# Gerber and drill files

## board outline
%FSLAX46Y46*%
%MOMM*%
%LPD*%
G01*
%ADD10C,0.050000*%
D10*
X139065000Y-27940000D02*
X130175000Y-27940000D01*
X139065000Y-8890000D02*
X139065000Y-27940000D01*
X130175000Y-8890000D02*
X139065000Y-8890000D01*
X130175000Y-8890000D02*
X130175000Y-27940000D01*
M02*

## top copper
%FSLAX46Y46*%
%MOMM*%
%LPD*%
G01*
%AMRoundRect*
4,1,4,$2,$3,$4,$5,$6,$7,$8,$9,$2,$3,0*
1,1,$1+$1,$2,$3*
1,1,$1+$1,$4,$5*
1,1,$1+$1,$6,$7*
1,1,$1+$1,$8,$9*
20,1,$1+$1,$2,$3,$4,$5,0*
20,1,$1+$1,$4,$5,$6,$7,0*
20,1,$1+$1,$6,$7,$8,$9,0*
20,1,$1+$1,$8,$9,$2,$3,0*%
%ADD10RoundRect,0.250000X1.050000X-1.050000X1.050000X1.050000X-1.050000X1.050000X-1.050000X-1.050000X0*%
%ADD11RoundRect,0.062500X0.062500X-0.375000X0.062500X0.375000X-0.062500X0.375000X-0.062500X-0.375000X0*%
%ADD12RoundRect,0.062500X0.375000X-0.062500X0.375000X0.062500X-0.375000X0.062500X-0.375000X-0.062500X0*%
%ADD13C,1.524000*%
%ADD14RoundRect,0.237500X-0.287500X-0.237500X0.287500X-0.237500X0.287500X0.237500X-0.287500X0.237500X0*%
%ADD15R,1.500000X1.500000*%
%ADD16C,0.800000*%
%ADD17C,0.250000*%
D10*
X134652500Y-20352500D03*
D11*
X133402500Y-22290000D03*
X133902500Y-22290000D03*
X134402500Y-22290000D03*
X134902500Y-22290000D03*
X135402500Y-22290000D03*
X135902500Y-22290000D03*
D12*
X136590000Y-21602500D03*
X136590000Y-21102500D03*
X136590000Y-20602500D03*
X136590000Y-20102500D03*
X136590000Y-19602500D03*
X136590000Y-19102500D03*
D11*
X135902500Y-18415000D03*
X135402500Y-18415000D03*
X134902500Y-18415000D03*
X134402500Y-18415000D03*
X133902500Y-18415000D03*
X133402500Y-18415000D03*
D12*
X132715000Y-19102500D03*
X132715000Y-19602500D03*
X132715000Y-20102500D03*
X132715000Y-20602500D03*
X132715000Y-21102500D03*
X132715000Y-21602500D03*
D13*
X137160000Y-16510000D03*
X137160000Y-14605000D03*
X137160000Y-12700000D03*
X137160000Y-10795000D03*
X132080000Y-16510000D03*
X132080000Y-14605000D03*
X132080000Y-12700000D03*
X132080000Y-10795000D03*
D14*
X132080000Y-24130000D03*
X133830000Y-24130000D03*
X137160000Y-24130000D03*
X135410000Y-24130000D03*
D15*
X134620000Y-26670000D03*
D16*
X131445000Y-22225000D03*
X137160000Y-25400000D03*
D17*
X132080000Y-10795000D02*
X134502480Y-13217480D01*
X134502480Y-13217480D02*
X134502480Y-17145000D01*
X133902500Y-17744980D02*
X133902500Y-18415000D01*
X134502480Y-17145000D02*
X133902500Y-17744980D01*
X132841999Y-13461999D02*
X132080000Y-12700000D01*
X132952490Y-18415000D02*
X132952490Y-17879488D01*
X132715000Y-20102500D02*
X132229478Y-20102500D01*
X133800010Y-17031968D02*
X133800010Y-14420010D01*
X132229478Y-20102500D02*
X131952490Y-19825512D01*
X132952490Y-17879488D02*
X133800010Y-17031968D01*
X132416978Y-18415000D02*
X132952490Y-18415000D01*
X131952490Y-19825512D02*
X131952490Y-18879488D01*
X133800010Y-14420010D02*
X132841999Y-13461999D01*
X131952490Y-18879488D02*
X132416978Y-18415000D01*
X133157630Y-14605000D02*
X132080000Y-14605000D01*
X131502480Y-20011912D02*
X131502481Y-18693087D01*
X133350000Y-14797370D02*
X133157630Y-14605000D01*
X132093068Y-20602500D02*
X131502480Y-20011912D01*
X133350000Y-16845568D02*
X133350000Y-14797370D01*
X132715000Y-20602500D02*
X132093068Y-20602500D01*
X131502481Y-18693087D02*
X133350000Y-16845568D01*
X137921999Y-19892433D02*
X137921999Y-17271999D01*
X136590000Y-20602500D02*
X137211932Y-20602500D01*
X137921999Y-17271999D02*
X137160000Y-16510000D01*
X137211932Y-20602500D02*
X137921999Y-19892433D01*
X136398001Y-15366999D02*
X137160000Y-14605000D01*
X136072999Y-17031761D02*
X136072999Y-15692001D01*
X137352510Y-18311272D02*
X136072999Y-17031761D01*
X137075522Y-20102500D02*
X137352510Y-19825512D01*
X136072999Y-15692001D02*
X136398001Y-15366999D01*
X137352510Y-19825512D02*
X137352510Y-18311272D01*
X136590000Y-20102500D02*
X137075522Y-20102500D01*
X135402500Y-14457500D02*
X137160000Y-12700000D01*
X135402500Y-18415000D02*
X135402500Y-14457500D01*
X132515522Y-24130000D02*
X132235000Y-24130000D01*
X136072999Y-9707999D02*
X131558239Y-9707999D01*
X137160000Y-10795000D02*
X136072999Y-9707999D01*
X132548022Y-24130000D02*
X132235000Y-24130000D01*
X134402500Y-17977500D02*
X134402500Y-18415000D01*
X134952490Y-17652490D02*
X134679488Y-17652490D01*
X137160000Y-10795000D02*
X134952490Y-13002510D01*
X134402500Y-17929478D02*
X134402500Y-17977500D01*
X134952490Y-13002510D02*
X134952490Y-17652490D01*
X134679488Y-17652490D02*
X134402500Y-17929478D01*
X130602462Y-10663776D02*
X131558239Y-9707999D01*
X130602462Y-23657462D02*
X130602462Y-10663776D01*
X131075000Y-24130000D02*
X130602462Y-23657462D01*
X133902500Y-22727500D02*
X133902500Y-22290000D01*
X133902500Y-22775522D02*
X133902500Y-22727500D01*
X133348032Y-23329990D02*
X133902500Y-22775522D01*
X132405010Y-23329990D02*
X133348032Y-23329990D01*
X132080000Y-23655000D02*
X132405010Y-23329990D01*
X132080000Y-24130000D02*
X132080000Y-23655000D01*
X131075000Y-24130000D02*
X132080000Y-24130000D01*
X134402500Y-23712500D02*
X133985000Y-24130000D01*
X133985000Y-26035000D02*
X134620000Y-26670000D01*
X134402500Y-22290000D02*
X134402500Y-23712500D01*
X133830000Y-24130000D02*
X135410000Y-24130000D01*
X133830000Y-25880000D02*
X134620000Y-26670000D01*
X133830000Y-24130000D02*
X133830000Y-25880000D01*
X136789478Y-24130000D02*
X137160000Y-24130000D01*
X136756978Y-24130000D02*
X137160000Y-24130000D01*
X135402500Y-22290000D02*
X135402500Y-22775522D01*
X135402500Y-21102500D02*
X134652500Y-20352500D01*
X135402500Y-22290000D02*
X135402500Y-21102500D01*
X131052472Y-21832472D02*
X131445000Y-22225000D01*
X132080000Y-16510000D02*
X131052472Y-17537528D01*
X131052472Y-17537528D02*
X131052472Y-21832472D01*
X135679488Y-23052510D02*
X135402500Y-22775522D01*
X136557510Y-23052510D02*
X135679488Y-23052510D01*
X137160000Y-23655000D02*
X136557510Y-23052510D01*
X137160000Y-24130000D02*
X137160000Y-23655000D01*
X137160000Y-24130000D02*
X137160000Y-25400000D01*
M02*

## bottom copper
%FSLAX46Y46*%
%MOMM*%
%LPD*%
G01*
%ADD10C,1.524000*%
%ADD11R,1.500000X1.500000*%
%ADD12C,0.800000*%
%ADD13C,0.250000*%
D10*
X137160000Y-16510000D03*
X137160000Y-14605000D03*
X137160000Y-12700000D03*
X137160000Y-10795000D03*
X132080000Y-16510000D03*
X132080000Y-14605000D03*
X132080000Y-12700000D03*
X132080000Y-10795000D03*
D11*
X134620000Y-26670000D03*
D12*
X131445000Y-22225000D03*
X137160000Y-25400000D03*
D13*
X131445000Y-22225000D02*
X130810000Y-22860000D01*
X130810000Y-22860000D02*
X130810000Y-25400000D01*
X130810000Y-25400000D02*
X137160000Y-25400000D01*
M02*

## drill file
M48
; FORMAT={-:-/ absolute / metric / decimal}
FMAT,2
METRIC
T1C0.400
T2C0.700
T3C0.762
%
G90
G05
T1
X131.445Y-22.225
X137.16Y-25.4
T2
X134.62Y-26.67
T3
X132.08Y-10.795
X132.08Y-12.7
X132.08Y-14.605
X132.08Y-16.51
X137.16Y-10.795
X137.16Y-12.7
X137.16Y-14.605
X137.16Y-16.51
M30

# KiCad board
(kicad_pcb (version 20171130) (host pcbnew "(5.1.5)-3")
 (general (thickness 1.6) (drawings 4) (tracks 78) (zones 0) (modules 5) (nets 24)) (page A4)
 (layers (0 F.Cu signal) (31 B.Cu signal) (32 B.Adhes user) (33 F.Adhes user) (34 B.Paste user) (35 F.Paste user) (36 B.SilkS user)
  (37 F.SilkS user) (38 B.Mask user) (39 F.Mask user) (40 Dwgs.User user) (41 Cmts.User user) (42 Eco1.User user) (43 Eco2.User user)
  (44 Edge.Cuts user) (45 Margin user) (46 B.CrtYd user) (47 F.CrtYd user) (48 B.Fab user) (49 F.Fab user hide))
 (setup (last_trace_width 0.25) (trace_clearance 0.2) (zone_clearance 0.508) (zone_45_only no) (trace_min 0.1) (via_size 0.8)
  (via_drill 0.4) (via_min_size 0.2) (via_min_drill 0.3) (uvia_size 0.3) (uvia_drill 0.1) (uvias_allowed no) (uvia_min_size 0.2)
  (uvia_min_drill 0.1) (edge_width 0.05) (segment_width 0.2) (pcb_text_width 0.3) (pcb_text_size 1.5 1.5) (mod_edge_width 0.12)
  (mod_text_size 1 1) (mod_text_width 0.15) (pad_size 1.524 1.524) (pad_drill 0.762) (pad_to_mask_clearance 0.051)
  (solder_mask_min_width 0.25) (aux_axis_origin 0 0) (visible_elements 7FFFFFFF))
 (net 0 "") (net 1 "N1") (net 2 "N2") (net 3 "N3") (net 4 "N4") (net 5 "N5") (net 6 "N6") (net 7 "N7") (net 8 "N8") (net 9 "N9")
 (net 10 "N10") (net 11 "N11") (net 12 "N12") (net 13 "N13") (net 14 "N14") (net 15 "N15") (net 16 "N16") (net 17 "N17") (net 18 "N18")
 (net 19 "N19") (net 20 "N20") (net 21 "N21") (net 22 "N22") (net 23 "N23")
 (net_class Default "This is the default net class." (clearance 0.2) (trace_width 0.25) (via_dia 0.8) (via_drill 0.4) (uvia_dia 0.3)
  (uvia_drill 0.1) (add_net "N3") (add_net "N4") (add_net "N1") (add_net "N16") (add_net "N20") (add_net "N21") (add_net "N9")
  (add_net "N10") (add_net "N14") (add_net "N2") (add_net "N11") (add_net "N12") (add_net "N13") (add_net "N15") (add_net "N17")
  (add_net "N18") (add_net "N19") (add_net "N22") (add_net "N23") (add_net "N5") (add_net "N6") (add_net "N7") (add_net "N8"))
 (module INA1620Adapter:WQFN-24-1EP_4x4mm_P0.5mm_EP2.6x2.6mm (layer F.Cu) (at 134.6525 20.3525 90)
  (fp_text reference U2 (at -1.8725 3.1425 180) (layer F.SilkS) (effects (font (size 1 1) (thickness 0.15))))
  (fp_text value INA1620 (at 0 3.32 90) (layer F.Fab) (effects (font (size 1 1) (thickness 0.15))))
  (pad 25 smd roundrect (at 0 0 90) (size 2.6 2.6) (layers F.Cu F.Mask) (roundrect_rratio 0.096154) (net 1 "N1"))
  (pad "" smd roundrect (at -0.65 -0.65 90) (size 1.05 1.05) (layers F.Paste) (roundrect_rratio 0.238095))
  (pad "" smd roundrect (at -0.65 0.65 90) (size 1.05 1.05) (layers F.Paste) (roundrect_rratio 0.238095))
  (pad "" smd roundrect (at 0.65 -0.65 90) (size 1.05 1.05) (layers F.Paste) (roundrect_rratio 0.238095))
  (pad "" smd roundrect (at 0.65 0.65 90) (size 1.05 1.05) (layers F.Paste) (roundrect_rratio 0.238095))
  (pad 1 smd roundrect (at -1.9375 -1.25 90) (size 0.875 0.25) (layers F.Cu F.Paste F.Mask) (roundrect_rratio 0.25) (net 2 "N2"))
  (pad 2 smd roundrect (at -1.9375 -0.75 90) (size 0.875 0.25) (layers F.Cu F.Paste F.Mask) (roundrect_rratio 0.25) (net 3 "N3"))
  (pad 3 smd roundrect (at -1.9375 -0.25 90) (size 0.875 0.25) (layers F.Cu F.Paste F.Mask) (roundrect_rratio 0.25) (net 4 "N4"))
  (pad 4 smd roundrect (at -1.9375 0.25 90) (size 0.875 0.25) (layers F.Cu F.Paste F.Mask) (roundrect_rratio 0.25) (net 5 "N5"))
  (pad 5 smd roundrect (at -1.9375 0.75 90) (size 0.875 0.25) (layers F.Cu F.Paste F.Mask) (roundrect_rratio 0.25) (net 1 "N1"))
  (pad 6 smd roundrect (at -1.9375 1.25 90) (size 0.875 0.25) (layers F.Cu F.Paste F.Mask) (roundrect_rratio 0.25) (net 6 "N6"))
  (pad 7 smd roundrect (at -1.25 1.9375 90) (size 0.25 0.875) (layers F.Cu F.Paste F.Mask) (roundrect_rratio 0.25) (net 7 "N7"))
  (pad 8 smd roundrect (at -0.75 1.9375 90) (size 0.25 0.875) (layers F.Cu F.Paste F.Mask) (roundrect_rratio 0.25) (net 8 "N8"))
  (pad 9 smd roundrect (at -0.25 1.9375 90) (size 0.25 0.875) (layers F.Cu F.Paste F.Mask) (roundrect_rratio 0.25) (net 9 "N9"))
  (pad 10 smd roundrect (at 0.25 1.9375 90) (size 0.25 0.875) (layers F.Cu F.Paste F.Mask) (roundrect_rratio 0.25) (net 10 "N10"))
  (pad 11 smd roundrect (at 0.75 1.9375 90) (size 0.25 0.875) (layers F.Cu F.Paste F.Mask) (roundrect_rratio 0.25) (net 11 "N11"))
  (pad 12 smd roundrect (at 1.25 1.9375 90) (size 0.25 0.875) (layers F.Cu F.Paste F.Mask) (roundrect_rratio 0.25) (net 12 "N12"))
  (pad 13 smd roundrect (at 1.9375 1.25 90) (size 0.875 0.25) (layers F.Cu F.Paste F.Mask) (roundrect_rratio 0.25) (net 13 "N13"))
  (pad 14 smd roundrect (at 1.9375 0.75 90) (size 0.875 0.25) (layers F.Cu F.Paste F.Mask) (roundrect_rratio 0.25) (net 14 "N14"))
  (pad 15 smd roundrect (at 1.9375 0.25 90) (size 0.875 0.25) (layers F.Cu F.Paste F.Mask) (roundrect_rratio 0.25) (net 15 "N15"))
  (pad 16 smd roundrect (at 1.9375 -0.25 90) (size 0.875 0.25) (layers F.Cu F.Paste F.Mask) (roundrect_rratio 0.25) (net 3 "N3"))
  (pad 17 smd roundrect (at 1.9375 -0.75 90) (size 0.875 0.25) (layers F.Cu F.Paste F.Mask) (roundrect_rratio 0.25) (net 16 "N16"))
  (pad 18 smd roundrect (at 1.9375 -1.25 90) (size 0.875 0.25) (layers F.Cu F.Paste F.Mask) (roundrect_rratio 0.25) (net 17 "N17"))
  (pad 19 smd roundrect (at 1.25 -1.9375 90) (size 0.25 0.875) (layers F.Cu F.Paste F.Mask) (roundrect_rratio 0.25) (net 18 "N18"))
  (pad 20 smd roundrect (at 0.75 -1.9375 90) (size 0.25 0.875) (layers F.Cu F.Paste F.Mask) (roundrect_rratio 0.25) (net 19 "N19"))
  (pad 21 smd roundrect (at 0.25 -1.9375 90) (size 0.25 0.875) (layers F.Cu F.Paste F.Mask) (roundrect_rratio 0.25) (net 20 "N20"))
  (pad 22 smd roundrect (at -0.25 -1.9375 90) (size 0.25 0.875) (layers F.Cu F.Paste F.Mask) (roundrect_rratio 0.25) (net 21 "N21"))
  (pad 23 smd roundrect (at -0.75 -1.9375 90) (size 0.25 0.875) (layers F.Cu F.Paste F.Mask) (roundrect_rratio 0.25) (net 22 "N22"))
  (pad 24 smd roundrect (at -1.25 -1.9375 90) (size 0.25 0.875) (layers F.Cu F.Paste F.Mask) (roundrect_rratio 0.25) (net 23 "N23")))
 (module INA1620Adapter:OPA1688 (layer F.Cu) (at 134.62 13.97)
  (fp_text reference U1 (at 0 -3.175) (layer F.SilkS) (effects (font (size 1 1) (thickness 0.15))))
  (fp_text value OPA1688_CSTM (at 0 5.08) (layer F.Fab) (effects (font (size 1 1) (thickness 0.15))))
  (pad 5 thru_hole circle (at 2.54 2.54) (size 1.524 1.524) (drill 0.762) (layers *.Cu *.Mask) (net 9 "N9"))
  (pad 6 thru_hole circle (at 2.54 0.635) (size 1.524 1.524) (drill 0.762) (layers *.Cu *.Mask) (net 10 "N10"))
  (pad 7 thru_hole circle (at 2.54 -1.27) (size 1.524 1.524) (drill 0.762) (layers *.Cu *.Mask) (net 14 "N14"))
  (pad 8 thru_hole circle (at 2.54 -3.175) (size 1.524 1.524) (drill 0.762) (layers *.Cu *.Mask) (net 3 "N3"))
  (pad 4 thru_hole circle (at -2.54 2.54) (size 1.524 1.524) (drill 0.762) (layers *.Cu *.Mask) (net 1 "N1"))
  (pad 3 thru_hole circle (at -2.54 0.635) (size 1.524 1.524) (drill 0.762) (layers *.Cu *.Mask) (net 21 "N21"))
  (pad 2 thru_hole circle (at -2.54 -1.27) (size 1.524 1.524) (drill 0.762) (layers *.Cu *.Mask) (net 20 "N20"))
  (pad 1 thru_hole circle (at -2.54 -3.175) (size 1.524 1.524) (drill 0.762) (layers *.Cu *.Mask) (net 16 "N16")))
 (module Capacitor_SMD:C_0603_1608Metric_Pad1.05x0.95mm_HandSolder (layer F.Cu) (at 132.955 24.13)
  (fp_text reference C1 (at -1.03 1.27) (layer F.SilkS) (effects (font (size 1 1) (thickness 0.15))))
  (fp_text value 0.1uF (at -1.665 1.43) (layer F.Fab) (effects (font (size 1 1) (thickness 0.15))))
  (pad 1 smd roundrect (at -0.875 0) (size 1.05 0.95) (layers F.Cu F.Paste F.Mask) (roundrect_rratio 0.25) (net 3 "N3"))
  (pad 2 smd roundrect (at 0.875 0) (size 1.05 0.95) (layers F.Cu F.Paste F.Mask) (roundrect_rratio 0.25) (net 4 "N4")))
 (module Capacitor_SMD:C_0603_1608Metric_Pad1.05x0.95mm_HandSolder (layer F.Cu) (at 136.285 24.13)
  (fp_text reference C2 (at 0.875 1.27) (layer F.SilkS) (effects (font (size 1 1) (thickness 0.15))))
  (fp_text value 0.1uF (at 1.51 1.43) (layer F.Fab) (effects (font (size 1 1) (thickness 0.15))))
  (pad 2 smd roundrect (at 0.875 0) (size 1.05 0.95) (layers F.Cu F.Paste F.Mask) (roundrect_rratio 0.25) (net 1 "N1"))
  (pad 1 smd roundrect (at -0.875 0) (size 1.05 0.95) (layers F.Cu F.Paste F.Mask) (roundrect_rratio 0.25) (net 4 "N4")))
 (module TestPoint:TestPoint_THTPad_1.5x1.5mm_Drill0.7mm (layer F.Cu) (at 134.62 26.67)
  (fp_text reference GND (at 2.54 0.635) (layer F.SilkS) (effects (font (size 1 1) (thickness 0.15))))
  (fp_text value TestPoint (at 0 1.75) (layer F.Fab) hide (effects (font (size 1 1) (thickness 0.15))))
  (pad 1 thru_hole rect (at 0 0) (size 1.5 1.5) (drill 0.7) (layers *.Cu *.Mask) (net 4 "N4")))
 (gr_line (start 139.065 27.94) (end 130.175 27.94) (layer Edge.Cuts) (width 0.05))
 (gr_line (start 139.065 8.89) (end 139.065 27.94) (layer Edge.Cuts) (width 0.05))
 (gr_line (start 130.175 8.89) (end 139.065 8.89) (layer Edge.Cuts) (width 0.05))
 (gr_line (start 130.175 8.89) (end 130.175 27.94) (layer Edge.Cuts) (width 0.05))
 (segment (start 132.08 10.795) (end 134.50248 13.21748) (width 0.25) (layer F.Cu) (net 16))
 (segment (start 134.50248 13.21748) (end 134.50248 17.145) (width 0.25) (layer F.Cu) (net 16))
 (segment (start 133.9025 17.74498) (end 133.9025 18.415) (width 0.25) (layer F.Cu) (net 16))
 (segment (start 134.50248 17.145) (end 133.9025 17.74498) (width 0.25) (layer F.Cu) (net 16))
 (segment (start 132.841999 13.461999) (end 132.08 12.7) (width 0.25) (layer F.Cu) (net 20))
 (segment (start 132.95249 18.415) (end 132.95249 17.879488) (width 0.25) (layer F.Cu) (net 20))
 (segment (start 132.715 20.1025) (end 132.229478 20.1025) (width 0.25) (layer F.Cu) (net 20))
 (segment (start 133.80001 17.031968) (end 133.80001 14.42001) (width 0.25) (layer F.Cu) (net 20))
 (segment (start 132.229478 20.1025) (end 131.95249 19.825512) (width 0.25) (layer F.Cu) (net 20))
 (segment (start 132.95249 17.879488) (end 133.80001 17.031968) (width 0.25) (layer F.Cu) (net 20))
 (segment (start 132.416978 18.415) (end 132.95249 18.415) (width 0.25) (layer F.Cu) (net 20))
 (segment (start 131.95249 19.825512) (end 131.95249 18.879488) (width 0.25) (layer F.Cu) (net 20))
 (segment (start 133.80001 14.42001) (end 132.841999 13.461999) (width 0.25) (layer F.Cu) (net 20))
 (segment (start 131.95249 18.879488) (end 132.416978 18.415) (width 0.25) (layer F.Cu) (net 20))
 (segment (start 133.15763 14.605) (end 132.08 14.605) (width 0.25) (layer F.Cu) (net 21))
 (segment (start 131.50248 20.011912) (end 131.502481 18.693087) (width 0.25) (layer F.Cu) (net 21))
 (segment (start 133.35 14.79737) (end 133.15763 14.605) (width 0.25) (layer F.Cu) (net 21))
 (segment (start 132.093068 20.6025) (end 131.50248 20.011912) (width 0.25) (layer F.Cu) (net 21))
 (segment (start 133.35 16.845568) (end 133.35 14.79737) (width 0.25) (layer F.Cu) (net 21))
 (segment (start 132.715 20.6025) (end 132.093068 20.6025) (width 0.25) (layer F.Cu) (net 21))
 (segment (start 131.502481 18.693087) (end 133.35 16.845568) (width 0.25) (layer F.Cu) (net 21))
 (segment (start 137.921999 19.892433) (end 137.921999 17.271999) (width 0.25) (layer F.Cu) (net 9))
 (segment (start 136.59 20.6025) (end 137.211932 20.6025) (width 0.25) (layer F.Cu) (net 9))
 (segment (start 137.921999 17.271999) (end 137.16 16.51) (width 0.25) (layer F.Cu) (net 9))
 (segment (start 137.211932 20.6025) (end 137.921999 19.892433) (width 0.25) (layer F.Cu) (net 9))
 (segment (start 136.398001 15.366999) (end 137.16 14.605) (width 0.25) (layer F.Cu) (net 10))
 (segment (start 136.072999 17.031761) (end 136.072999 15.692001) (width 0.25) (layer F.Cu) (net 10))
 (segment (start 137.35251 18.311272) (end 136.072999 17.031761) (width 0.25) (layer F.Cu) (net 10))
 (segment (start 137.075522 20.1025) (end 137.35251 19.825512) (width 0.25) (layer F.Cu) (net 10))
 (segment (start 136.072999 15.692001) (end 136.398001 15.366999) (width 0.25) (layer F.Cu) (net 10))
 (segment (start 137.35251 19.825512) (end 137.35251 18.311272) (width 0.25) (layer F.Cu) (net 10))
 (segment (start 136.59 20.1025) (end 137.075522 20.1025) (width 0.25) (layer F.Cu) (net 10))
 (segment (start 135.4025 14.4575) (end 137.16 12.7) (width 0.25) (layer F.Cu) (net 14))
 (segment (start 135.4025 18.415) (end 135.4025 14.4575) (width 0.25) (layer F.Cu) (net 14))
 (segment (start 132.515522 24.13) (end 132.235 24.13) (width 0.25) (layer F.Cu) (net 3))
 (segment (start 136.072999 9.707999) (end 131.558239 9.707999) (width 0.25) (layer F.Cu) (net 3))
 (segment (start 137.16 10.795) (end 136.072999 9.707999) (width 0.25) (layer F.Cu) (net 3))
 (segment (start 132.548022 24.13) (end 132.235 24.13) (width 0.25) (layer F.Cu) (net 3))
 (segment (start 134.4025 17.9775) (end 134.4025 18.415) (width 0.25) (layer F.Cu) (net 3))
 (segment (start 134.95249 17.65249) (end 134.679488 17.65249) (width 0.25) (layer F.Cu) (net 3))
 (segment (start 137.16 10.795) (end 134.95249 13.00251) (width 0.25) (layer F.Cu) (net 3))
 (segment (start 134.4025 17.929478) (end 134.4025 17.9775) (width 0.25) (layer F.Cu) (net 3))
 (segment (start 134.95249 13.00251) (end 134.95249 17.65249) (width 0.25) (layer F.Cu) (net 3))
 (segment (start 134.679488 17.65249) (end 134.4025 17.929478) (width 0.25) (layer F.Cu) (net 3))
 (segment (start 130.602462 10.663776) (end 131.558239 9.707999) (width 0.25) (layer F.Cu) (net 3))
 (segment (start 130.602462 23.657462) (end 130.602462 10.663776) (width 0.25) (layer F.Cu) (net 3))
 (segment (start 131.075 24.13) (end 130.602462 23.657462) (width 0.25) (layer F.Cu) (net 3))
 (segment (start 133.9025 22.7275) (end 133.9025 22.29) (width 0.25) (layer F.Cu) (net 3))
 (segment (start 133.9025 22.775522) (end 133.9025 22.7275) (width 0.25) (layer F.Cu) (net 3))
 (segment (start 133.348032 23.32999) (end 133.9025 22.775522) (width 0.25) (layer F.Cu) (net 3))
 (segment (start 132.40501 23.32999) (end 133.348032 23.32999) (width 0.25) (layer F.Cu) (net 3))
 (segment (start 132.08 23.655) (end 132.40501 23.32999) (width 0.25) (layer F.Cu) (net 3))
 (segment (start 132.08 24.13) (end 132.08 23.655) (width 0.25) (layer F.Cu) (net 3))
 (segment (start 131.075 24.13) (end 132.08 24.13) (width 0.25) (layer F.Cu) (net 3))
 (segment (start 134.4025 23.7125) (end 133.985 24.13) (width 0.25) (layer F.Cu) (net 4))
 (segment (start 133.985 26.035) (end 134.62 26.67) (width 0.25) (layer F.Cu) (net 4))
 (segment (start 134.4025 22.29) (end 134.4025 23.7125) (width 0.25) (layer F.Cu) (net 4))
 (segment (start 133.83 24.13) (end 135.41 24.13) (width 0.25) (layer F.Cu) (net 4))
 (segment (start 133.83 25.88) (end 134.62 26.67) (width 0.25) (layer F.Cu) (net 4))
 (segment (start 133.83 24.13) (end 133.83 25.88) (width 0.25) (layer F.Cu) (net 4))
 (segment (start 136.789478 24.13) (end 137.16 24.13) (width 0.25) (layer F.Cu) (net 1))
 (segment (start 136.756978 24.13) (end 137.16 24.13) (width 0.25) (layer F.Cu) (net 1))
 (segment (start 135.4025 22.29) (end 135.4025 22.775522) (width 0.25) (layer F.Cu) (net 1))
 (segment (start 135.4025 21.1025) (end 134.6525 20.3525) (width 0.25) (layer F.Cu) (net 1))
 (segment (start 135.4025 22.29) (end 135.4025 21.1025) (width 0.25) (layer F.Cu) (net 1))
 (segment (start 131.052472 21.832472) (end 131.445 22.225) (width 0.25) (layer F.Cu) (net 1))
 (segment (start 132.08 16.51) (end 131.052472 17.537528) (width 0.25) (layer F.Cu) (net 1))
 (via (at 131.445 22.225) (size 0.8) (drill 0.4) (layers F.Cu B.Cu) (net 1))
 (segment (start 131.052472 17.537528) (end 131.052472 21.832472) (width 0.25) (layer F.Cu) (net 1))
 (segment (start 131.445 22.225) (end 130.81 22.86) (width 0.25) (layer B.Cu) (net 1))
 (segment (start 130.81 22.86) (end 130.81 25.4) (width 0.25) (layer B.Cu) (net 1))
 (via (at 137.16 25.4) (size 0.8) (drill 0.4) (layers F.Cu B.Cu) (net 1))
 (segment (start 130.81 25.4) (end 137.16 25.4) (width 0.25) (layer B.Cu) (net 1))
 (segment (start 135.679488 23.05251) (end 135.4025 22.775522) (width 0.25) (layer F.Cu) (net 1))
 (segment (start 136.55751 23.05251) (end 135.679488 23.05251) (width 0.25) (layer F.Cu) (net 1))
 (segment (start 137.16 23.655) (end 136.55751 23.05251) (width 0.25) (layer F.Cu) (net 1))
 (segment (start 137.16 24.13) (end 137.16 23.655) (width 0.25) (layer F.Cu) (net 1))
 (segment (start 137.16 24.13) (end 137.16 25.4) (width 0.25) (layer F.Cu) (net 1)))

